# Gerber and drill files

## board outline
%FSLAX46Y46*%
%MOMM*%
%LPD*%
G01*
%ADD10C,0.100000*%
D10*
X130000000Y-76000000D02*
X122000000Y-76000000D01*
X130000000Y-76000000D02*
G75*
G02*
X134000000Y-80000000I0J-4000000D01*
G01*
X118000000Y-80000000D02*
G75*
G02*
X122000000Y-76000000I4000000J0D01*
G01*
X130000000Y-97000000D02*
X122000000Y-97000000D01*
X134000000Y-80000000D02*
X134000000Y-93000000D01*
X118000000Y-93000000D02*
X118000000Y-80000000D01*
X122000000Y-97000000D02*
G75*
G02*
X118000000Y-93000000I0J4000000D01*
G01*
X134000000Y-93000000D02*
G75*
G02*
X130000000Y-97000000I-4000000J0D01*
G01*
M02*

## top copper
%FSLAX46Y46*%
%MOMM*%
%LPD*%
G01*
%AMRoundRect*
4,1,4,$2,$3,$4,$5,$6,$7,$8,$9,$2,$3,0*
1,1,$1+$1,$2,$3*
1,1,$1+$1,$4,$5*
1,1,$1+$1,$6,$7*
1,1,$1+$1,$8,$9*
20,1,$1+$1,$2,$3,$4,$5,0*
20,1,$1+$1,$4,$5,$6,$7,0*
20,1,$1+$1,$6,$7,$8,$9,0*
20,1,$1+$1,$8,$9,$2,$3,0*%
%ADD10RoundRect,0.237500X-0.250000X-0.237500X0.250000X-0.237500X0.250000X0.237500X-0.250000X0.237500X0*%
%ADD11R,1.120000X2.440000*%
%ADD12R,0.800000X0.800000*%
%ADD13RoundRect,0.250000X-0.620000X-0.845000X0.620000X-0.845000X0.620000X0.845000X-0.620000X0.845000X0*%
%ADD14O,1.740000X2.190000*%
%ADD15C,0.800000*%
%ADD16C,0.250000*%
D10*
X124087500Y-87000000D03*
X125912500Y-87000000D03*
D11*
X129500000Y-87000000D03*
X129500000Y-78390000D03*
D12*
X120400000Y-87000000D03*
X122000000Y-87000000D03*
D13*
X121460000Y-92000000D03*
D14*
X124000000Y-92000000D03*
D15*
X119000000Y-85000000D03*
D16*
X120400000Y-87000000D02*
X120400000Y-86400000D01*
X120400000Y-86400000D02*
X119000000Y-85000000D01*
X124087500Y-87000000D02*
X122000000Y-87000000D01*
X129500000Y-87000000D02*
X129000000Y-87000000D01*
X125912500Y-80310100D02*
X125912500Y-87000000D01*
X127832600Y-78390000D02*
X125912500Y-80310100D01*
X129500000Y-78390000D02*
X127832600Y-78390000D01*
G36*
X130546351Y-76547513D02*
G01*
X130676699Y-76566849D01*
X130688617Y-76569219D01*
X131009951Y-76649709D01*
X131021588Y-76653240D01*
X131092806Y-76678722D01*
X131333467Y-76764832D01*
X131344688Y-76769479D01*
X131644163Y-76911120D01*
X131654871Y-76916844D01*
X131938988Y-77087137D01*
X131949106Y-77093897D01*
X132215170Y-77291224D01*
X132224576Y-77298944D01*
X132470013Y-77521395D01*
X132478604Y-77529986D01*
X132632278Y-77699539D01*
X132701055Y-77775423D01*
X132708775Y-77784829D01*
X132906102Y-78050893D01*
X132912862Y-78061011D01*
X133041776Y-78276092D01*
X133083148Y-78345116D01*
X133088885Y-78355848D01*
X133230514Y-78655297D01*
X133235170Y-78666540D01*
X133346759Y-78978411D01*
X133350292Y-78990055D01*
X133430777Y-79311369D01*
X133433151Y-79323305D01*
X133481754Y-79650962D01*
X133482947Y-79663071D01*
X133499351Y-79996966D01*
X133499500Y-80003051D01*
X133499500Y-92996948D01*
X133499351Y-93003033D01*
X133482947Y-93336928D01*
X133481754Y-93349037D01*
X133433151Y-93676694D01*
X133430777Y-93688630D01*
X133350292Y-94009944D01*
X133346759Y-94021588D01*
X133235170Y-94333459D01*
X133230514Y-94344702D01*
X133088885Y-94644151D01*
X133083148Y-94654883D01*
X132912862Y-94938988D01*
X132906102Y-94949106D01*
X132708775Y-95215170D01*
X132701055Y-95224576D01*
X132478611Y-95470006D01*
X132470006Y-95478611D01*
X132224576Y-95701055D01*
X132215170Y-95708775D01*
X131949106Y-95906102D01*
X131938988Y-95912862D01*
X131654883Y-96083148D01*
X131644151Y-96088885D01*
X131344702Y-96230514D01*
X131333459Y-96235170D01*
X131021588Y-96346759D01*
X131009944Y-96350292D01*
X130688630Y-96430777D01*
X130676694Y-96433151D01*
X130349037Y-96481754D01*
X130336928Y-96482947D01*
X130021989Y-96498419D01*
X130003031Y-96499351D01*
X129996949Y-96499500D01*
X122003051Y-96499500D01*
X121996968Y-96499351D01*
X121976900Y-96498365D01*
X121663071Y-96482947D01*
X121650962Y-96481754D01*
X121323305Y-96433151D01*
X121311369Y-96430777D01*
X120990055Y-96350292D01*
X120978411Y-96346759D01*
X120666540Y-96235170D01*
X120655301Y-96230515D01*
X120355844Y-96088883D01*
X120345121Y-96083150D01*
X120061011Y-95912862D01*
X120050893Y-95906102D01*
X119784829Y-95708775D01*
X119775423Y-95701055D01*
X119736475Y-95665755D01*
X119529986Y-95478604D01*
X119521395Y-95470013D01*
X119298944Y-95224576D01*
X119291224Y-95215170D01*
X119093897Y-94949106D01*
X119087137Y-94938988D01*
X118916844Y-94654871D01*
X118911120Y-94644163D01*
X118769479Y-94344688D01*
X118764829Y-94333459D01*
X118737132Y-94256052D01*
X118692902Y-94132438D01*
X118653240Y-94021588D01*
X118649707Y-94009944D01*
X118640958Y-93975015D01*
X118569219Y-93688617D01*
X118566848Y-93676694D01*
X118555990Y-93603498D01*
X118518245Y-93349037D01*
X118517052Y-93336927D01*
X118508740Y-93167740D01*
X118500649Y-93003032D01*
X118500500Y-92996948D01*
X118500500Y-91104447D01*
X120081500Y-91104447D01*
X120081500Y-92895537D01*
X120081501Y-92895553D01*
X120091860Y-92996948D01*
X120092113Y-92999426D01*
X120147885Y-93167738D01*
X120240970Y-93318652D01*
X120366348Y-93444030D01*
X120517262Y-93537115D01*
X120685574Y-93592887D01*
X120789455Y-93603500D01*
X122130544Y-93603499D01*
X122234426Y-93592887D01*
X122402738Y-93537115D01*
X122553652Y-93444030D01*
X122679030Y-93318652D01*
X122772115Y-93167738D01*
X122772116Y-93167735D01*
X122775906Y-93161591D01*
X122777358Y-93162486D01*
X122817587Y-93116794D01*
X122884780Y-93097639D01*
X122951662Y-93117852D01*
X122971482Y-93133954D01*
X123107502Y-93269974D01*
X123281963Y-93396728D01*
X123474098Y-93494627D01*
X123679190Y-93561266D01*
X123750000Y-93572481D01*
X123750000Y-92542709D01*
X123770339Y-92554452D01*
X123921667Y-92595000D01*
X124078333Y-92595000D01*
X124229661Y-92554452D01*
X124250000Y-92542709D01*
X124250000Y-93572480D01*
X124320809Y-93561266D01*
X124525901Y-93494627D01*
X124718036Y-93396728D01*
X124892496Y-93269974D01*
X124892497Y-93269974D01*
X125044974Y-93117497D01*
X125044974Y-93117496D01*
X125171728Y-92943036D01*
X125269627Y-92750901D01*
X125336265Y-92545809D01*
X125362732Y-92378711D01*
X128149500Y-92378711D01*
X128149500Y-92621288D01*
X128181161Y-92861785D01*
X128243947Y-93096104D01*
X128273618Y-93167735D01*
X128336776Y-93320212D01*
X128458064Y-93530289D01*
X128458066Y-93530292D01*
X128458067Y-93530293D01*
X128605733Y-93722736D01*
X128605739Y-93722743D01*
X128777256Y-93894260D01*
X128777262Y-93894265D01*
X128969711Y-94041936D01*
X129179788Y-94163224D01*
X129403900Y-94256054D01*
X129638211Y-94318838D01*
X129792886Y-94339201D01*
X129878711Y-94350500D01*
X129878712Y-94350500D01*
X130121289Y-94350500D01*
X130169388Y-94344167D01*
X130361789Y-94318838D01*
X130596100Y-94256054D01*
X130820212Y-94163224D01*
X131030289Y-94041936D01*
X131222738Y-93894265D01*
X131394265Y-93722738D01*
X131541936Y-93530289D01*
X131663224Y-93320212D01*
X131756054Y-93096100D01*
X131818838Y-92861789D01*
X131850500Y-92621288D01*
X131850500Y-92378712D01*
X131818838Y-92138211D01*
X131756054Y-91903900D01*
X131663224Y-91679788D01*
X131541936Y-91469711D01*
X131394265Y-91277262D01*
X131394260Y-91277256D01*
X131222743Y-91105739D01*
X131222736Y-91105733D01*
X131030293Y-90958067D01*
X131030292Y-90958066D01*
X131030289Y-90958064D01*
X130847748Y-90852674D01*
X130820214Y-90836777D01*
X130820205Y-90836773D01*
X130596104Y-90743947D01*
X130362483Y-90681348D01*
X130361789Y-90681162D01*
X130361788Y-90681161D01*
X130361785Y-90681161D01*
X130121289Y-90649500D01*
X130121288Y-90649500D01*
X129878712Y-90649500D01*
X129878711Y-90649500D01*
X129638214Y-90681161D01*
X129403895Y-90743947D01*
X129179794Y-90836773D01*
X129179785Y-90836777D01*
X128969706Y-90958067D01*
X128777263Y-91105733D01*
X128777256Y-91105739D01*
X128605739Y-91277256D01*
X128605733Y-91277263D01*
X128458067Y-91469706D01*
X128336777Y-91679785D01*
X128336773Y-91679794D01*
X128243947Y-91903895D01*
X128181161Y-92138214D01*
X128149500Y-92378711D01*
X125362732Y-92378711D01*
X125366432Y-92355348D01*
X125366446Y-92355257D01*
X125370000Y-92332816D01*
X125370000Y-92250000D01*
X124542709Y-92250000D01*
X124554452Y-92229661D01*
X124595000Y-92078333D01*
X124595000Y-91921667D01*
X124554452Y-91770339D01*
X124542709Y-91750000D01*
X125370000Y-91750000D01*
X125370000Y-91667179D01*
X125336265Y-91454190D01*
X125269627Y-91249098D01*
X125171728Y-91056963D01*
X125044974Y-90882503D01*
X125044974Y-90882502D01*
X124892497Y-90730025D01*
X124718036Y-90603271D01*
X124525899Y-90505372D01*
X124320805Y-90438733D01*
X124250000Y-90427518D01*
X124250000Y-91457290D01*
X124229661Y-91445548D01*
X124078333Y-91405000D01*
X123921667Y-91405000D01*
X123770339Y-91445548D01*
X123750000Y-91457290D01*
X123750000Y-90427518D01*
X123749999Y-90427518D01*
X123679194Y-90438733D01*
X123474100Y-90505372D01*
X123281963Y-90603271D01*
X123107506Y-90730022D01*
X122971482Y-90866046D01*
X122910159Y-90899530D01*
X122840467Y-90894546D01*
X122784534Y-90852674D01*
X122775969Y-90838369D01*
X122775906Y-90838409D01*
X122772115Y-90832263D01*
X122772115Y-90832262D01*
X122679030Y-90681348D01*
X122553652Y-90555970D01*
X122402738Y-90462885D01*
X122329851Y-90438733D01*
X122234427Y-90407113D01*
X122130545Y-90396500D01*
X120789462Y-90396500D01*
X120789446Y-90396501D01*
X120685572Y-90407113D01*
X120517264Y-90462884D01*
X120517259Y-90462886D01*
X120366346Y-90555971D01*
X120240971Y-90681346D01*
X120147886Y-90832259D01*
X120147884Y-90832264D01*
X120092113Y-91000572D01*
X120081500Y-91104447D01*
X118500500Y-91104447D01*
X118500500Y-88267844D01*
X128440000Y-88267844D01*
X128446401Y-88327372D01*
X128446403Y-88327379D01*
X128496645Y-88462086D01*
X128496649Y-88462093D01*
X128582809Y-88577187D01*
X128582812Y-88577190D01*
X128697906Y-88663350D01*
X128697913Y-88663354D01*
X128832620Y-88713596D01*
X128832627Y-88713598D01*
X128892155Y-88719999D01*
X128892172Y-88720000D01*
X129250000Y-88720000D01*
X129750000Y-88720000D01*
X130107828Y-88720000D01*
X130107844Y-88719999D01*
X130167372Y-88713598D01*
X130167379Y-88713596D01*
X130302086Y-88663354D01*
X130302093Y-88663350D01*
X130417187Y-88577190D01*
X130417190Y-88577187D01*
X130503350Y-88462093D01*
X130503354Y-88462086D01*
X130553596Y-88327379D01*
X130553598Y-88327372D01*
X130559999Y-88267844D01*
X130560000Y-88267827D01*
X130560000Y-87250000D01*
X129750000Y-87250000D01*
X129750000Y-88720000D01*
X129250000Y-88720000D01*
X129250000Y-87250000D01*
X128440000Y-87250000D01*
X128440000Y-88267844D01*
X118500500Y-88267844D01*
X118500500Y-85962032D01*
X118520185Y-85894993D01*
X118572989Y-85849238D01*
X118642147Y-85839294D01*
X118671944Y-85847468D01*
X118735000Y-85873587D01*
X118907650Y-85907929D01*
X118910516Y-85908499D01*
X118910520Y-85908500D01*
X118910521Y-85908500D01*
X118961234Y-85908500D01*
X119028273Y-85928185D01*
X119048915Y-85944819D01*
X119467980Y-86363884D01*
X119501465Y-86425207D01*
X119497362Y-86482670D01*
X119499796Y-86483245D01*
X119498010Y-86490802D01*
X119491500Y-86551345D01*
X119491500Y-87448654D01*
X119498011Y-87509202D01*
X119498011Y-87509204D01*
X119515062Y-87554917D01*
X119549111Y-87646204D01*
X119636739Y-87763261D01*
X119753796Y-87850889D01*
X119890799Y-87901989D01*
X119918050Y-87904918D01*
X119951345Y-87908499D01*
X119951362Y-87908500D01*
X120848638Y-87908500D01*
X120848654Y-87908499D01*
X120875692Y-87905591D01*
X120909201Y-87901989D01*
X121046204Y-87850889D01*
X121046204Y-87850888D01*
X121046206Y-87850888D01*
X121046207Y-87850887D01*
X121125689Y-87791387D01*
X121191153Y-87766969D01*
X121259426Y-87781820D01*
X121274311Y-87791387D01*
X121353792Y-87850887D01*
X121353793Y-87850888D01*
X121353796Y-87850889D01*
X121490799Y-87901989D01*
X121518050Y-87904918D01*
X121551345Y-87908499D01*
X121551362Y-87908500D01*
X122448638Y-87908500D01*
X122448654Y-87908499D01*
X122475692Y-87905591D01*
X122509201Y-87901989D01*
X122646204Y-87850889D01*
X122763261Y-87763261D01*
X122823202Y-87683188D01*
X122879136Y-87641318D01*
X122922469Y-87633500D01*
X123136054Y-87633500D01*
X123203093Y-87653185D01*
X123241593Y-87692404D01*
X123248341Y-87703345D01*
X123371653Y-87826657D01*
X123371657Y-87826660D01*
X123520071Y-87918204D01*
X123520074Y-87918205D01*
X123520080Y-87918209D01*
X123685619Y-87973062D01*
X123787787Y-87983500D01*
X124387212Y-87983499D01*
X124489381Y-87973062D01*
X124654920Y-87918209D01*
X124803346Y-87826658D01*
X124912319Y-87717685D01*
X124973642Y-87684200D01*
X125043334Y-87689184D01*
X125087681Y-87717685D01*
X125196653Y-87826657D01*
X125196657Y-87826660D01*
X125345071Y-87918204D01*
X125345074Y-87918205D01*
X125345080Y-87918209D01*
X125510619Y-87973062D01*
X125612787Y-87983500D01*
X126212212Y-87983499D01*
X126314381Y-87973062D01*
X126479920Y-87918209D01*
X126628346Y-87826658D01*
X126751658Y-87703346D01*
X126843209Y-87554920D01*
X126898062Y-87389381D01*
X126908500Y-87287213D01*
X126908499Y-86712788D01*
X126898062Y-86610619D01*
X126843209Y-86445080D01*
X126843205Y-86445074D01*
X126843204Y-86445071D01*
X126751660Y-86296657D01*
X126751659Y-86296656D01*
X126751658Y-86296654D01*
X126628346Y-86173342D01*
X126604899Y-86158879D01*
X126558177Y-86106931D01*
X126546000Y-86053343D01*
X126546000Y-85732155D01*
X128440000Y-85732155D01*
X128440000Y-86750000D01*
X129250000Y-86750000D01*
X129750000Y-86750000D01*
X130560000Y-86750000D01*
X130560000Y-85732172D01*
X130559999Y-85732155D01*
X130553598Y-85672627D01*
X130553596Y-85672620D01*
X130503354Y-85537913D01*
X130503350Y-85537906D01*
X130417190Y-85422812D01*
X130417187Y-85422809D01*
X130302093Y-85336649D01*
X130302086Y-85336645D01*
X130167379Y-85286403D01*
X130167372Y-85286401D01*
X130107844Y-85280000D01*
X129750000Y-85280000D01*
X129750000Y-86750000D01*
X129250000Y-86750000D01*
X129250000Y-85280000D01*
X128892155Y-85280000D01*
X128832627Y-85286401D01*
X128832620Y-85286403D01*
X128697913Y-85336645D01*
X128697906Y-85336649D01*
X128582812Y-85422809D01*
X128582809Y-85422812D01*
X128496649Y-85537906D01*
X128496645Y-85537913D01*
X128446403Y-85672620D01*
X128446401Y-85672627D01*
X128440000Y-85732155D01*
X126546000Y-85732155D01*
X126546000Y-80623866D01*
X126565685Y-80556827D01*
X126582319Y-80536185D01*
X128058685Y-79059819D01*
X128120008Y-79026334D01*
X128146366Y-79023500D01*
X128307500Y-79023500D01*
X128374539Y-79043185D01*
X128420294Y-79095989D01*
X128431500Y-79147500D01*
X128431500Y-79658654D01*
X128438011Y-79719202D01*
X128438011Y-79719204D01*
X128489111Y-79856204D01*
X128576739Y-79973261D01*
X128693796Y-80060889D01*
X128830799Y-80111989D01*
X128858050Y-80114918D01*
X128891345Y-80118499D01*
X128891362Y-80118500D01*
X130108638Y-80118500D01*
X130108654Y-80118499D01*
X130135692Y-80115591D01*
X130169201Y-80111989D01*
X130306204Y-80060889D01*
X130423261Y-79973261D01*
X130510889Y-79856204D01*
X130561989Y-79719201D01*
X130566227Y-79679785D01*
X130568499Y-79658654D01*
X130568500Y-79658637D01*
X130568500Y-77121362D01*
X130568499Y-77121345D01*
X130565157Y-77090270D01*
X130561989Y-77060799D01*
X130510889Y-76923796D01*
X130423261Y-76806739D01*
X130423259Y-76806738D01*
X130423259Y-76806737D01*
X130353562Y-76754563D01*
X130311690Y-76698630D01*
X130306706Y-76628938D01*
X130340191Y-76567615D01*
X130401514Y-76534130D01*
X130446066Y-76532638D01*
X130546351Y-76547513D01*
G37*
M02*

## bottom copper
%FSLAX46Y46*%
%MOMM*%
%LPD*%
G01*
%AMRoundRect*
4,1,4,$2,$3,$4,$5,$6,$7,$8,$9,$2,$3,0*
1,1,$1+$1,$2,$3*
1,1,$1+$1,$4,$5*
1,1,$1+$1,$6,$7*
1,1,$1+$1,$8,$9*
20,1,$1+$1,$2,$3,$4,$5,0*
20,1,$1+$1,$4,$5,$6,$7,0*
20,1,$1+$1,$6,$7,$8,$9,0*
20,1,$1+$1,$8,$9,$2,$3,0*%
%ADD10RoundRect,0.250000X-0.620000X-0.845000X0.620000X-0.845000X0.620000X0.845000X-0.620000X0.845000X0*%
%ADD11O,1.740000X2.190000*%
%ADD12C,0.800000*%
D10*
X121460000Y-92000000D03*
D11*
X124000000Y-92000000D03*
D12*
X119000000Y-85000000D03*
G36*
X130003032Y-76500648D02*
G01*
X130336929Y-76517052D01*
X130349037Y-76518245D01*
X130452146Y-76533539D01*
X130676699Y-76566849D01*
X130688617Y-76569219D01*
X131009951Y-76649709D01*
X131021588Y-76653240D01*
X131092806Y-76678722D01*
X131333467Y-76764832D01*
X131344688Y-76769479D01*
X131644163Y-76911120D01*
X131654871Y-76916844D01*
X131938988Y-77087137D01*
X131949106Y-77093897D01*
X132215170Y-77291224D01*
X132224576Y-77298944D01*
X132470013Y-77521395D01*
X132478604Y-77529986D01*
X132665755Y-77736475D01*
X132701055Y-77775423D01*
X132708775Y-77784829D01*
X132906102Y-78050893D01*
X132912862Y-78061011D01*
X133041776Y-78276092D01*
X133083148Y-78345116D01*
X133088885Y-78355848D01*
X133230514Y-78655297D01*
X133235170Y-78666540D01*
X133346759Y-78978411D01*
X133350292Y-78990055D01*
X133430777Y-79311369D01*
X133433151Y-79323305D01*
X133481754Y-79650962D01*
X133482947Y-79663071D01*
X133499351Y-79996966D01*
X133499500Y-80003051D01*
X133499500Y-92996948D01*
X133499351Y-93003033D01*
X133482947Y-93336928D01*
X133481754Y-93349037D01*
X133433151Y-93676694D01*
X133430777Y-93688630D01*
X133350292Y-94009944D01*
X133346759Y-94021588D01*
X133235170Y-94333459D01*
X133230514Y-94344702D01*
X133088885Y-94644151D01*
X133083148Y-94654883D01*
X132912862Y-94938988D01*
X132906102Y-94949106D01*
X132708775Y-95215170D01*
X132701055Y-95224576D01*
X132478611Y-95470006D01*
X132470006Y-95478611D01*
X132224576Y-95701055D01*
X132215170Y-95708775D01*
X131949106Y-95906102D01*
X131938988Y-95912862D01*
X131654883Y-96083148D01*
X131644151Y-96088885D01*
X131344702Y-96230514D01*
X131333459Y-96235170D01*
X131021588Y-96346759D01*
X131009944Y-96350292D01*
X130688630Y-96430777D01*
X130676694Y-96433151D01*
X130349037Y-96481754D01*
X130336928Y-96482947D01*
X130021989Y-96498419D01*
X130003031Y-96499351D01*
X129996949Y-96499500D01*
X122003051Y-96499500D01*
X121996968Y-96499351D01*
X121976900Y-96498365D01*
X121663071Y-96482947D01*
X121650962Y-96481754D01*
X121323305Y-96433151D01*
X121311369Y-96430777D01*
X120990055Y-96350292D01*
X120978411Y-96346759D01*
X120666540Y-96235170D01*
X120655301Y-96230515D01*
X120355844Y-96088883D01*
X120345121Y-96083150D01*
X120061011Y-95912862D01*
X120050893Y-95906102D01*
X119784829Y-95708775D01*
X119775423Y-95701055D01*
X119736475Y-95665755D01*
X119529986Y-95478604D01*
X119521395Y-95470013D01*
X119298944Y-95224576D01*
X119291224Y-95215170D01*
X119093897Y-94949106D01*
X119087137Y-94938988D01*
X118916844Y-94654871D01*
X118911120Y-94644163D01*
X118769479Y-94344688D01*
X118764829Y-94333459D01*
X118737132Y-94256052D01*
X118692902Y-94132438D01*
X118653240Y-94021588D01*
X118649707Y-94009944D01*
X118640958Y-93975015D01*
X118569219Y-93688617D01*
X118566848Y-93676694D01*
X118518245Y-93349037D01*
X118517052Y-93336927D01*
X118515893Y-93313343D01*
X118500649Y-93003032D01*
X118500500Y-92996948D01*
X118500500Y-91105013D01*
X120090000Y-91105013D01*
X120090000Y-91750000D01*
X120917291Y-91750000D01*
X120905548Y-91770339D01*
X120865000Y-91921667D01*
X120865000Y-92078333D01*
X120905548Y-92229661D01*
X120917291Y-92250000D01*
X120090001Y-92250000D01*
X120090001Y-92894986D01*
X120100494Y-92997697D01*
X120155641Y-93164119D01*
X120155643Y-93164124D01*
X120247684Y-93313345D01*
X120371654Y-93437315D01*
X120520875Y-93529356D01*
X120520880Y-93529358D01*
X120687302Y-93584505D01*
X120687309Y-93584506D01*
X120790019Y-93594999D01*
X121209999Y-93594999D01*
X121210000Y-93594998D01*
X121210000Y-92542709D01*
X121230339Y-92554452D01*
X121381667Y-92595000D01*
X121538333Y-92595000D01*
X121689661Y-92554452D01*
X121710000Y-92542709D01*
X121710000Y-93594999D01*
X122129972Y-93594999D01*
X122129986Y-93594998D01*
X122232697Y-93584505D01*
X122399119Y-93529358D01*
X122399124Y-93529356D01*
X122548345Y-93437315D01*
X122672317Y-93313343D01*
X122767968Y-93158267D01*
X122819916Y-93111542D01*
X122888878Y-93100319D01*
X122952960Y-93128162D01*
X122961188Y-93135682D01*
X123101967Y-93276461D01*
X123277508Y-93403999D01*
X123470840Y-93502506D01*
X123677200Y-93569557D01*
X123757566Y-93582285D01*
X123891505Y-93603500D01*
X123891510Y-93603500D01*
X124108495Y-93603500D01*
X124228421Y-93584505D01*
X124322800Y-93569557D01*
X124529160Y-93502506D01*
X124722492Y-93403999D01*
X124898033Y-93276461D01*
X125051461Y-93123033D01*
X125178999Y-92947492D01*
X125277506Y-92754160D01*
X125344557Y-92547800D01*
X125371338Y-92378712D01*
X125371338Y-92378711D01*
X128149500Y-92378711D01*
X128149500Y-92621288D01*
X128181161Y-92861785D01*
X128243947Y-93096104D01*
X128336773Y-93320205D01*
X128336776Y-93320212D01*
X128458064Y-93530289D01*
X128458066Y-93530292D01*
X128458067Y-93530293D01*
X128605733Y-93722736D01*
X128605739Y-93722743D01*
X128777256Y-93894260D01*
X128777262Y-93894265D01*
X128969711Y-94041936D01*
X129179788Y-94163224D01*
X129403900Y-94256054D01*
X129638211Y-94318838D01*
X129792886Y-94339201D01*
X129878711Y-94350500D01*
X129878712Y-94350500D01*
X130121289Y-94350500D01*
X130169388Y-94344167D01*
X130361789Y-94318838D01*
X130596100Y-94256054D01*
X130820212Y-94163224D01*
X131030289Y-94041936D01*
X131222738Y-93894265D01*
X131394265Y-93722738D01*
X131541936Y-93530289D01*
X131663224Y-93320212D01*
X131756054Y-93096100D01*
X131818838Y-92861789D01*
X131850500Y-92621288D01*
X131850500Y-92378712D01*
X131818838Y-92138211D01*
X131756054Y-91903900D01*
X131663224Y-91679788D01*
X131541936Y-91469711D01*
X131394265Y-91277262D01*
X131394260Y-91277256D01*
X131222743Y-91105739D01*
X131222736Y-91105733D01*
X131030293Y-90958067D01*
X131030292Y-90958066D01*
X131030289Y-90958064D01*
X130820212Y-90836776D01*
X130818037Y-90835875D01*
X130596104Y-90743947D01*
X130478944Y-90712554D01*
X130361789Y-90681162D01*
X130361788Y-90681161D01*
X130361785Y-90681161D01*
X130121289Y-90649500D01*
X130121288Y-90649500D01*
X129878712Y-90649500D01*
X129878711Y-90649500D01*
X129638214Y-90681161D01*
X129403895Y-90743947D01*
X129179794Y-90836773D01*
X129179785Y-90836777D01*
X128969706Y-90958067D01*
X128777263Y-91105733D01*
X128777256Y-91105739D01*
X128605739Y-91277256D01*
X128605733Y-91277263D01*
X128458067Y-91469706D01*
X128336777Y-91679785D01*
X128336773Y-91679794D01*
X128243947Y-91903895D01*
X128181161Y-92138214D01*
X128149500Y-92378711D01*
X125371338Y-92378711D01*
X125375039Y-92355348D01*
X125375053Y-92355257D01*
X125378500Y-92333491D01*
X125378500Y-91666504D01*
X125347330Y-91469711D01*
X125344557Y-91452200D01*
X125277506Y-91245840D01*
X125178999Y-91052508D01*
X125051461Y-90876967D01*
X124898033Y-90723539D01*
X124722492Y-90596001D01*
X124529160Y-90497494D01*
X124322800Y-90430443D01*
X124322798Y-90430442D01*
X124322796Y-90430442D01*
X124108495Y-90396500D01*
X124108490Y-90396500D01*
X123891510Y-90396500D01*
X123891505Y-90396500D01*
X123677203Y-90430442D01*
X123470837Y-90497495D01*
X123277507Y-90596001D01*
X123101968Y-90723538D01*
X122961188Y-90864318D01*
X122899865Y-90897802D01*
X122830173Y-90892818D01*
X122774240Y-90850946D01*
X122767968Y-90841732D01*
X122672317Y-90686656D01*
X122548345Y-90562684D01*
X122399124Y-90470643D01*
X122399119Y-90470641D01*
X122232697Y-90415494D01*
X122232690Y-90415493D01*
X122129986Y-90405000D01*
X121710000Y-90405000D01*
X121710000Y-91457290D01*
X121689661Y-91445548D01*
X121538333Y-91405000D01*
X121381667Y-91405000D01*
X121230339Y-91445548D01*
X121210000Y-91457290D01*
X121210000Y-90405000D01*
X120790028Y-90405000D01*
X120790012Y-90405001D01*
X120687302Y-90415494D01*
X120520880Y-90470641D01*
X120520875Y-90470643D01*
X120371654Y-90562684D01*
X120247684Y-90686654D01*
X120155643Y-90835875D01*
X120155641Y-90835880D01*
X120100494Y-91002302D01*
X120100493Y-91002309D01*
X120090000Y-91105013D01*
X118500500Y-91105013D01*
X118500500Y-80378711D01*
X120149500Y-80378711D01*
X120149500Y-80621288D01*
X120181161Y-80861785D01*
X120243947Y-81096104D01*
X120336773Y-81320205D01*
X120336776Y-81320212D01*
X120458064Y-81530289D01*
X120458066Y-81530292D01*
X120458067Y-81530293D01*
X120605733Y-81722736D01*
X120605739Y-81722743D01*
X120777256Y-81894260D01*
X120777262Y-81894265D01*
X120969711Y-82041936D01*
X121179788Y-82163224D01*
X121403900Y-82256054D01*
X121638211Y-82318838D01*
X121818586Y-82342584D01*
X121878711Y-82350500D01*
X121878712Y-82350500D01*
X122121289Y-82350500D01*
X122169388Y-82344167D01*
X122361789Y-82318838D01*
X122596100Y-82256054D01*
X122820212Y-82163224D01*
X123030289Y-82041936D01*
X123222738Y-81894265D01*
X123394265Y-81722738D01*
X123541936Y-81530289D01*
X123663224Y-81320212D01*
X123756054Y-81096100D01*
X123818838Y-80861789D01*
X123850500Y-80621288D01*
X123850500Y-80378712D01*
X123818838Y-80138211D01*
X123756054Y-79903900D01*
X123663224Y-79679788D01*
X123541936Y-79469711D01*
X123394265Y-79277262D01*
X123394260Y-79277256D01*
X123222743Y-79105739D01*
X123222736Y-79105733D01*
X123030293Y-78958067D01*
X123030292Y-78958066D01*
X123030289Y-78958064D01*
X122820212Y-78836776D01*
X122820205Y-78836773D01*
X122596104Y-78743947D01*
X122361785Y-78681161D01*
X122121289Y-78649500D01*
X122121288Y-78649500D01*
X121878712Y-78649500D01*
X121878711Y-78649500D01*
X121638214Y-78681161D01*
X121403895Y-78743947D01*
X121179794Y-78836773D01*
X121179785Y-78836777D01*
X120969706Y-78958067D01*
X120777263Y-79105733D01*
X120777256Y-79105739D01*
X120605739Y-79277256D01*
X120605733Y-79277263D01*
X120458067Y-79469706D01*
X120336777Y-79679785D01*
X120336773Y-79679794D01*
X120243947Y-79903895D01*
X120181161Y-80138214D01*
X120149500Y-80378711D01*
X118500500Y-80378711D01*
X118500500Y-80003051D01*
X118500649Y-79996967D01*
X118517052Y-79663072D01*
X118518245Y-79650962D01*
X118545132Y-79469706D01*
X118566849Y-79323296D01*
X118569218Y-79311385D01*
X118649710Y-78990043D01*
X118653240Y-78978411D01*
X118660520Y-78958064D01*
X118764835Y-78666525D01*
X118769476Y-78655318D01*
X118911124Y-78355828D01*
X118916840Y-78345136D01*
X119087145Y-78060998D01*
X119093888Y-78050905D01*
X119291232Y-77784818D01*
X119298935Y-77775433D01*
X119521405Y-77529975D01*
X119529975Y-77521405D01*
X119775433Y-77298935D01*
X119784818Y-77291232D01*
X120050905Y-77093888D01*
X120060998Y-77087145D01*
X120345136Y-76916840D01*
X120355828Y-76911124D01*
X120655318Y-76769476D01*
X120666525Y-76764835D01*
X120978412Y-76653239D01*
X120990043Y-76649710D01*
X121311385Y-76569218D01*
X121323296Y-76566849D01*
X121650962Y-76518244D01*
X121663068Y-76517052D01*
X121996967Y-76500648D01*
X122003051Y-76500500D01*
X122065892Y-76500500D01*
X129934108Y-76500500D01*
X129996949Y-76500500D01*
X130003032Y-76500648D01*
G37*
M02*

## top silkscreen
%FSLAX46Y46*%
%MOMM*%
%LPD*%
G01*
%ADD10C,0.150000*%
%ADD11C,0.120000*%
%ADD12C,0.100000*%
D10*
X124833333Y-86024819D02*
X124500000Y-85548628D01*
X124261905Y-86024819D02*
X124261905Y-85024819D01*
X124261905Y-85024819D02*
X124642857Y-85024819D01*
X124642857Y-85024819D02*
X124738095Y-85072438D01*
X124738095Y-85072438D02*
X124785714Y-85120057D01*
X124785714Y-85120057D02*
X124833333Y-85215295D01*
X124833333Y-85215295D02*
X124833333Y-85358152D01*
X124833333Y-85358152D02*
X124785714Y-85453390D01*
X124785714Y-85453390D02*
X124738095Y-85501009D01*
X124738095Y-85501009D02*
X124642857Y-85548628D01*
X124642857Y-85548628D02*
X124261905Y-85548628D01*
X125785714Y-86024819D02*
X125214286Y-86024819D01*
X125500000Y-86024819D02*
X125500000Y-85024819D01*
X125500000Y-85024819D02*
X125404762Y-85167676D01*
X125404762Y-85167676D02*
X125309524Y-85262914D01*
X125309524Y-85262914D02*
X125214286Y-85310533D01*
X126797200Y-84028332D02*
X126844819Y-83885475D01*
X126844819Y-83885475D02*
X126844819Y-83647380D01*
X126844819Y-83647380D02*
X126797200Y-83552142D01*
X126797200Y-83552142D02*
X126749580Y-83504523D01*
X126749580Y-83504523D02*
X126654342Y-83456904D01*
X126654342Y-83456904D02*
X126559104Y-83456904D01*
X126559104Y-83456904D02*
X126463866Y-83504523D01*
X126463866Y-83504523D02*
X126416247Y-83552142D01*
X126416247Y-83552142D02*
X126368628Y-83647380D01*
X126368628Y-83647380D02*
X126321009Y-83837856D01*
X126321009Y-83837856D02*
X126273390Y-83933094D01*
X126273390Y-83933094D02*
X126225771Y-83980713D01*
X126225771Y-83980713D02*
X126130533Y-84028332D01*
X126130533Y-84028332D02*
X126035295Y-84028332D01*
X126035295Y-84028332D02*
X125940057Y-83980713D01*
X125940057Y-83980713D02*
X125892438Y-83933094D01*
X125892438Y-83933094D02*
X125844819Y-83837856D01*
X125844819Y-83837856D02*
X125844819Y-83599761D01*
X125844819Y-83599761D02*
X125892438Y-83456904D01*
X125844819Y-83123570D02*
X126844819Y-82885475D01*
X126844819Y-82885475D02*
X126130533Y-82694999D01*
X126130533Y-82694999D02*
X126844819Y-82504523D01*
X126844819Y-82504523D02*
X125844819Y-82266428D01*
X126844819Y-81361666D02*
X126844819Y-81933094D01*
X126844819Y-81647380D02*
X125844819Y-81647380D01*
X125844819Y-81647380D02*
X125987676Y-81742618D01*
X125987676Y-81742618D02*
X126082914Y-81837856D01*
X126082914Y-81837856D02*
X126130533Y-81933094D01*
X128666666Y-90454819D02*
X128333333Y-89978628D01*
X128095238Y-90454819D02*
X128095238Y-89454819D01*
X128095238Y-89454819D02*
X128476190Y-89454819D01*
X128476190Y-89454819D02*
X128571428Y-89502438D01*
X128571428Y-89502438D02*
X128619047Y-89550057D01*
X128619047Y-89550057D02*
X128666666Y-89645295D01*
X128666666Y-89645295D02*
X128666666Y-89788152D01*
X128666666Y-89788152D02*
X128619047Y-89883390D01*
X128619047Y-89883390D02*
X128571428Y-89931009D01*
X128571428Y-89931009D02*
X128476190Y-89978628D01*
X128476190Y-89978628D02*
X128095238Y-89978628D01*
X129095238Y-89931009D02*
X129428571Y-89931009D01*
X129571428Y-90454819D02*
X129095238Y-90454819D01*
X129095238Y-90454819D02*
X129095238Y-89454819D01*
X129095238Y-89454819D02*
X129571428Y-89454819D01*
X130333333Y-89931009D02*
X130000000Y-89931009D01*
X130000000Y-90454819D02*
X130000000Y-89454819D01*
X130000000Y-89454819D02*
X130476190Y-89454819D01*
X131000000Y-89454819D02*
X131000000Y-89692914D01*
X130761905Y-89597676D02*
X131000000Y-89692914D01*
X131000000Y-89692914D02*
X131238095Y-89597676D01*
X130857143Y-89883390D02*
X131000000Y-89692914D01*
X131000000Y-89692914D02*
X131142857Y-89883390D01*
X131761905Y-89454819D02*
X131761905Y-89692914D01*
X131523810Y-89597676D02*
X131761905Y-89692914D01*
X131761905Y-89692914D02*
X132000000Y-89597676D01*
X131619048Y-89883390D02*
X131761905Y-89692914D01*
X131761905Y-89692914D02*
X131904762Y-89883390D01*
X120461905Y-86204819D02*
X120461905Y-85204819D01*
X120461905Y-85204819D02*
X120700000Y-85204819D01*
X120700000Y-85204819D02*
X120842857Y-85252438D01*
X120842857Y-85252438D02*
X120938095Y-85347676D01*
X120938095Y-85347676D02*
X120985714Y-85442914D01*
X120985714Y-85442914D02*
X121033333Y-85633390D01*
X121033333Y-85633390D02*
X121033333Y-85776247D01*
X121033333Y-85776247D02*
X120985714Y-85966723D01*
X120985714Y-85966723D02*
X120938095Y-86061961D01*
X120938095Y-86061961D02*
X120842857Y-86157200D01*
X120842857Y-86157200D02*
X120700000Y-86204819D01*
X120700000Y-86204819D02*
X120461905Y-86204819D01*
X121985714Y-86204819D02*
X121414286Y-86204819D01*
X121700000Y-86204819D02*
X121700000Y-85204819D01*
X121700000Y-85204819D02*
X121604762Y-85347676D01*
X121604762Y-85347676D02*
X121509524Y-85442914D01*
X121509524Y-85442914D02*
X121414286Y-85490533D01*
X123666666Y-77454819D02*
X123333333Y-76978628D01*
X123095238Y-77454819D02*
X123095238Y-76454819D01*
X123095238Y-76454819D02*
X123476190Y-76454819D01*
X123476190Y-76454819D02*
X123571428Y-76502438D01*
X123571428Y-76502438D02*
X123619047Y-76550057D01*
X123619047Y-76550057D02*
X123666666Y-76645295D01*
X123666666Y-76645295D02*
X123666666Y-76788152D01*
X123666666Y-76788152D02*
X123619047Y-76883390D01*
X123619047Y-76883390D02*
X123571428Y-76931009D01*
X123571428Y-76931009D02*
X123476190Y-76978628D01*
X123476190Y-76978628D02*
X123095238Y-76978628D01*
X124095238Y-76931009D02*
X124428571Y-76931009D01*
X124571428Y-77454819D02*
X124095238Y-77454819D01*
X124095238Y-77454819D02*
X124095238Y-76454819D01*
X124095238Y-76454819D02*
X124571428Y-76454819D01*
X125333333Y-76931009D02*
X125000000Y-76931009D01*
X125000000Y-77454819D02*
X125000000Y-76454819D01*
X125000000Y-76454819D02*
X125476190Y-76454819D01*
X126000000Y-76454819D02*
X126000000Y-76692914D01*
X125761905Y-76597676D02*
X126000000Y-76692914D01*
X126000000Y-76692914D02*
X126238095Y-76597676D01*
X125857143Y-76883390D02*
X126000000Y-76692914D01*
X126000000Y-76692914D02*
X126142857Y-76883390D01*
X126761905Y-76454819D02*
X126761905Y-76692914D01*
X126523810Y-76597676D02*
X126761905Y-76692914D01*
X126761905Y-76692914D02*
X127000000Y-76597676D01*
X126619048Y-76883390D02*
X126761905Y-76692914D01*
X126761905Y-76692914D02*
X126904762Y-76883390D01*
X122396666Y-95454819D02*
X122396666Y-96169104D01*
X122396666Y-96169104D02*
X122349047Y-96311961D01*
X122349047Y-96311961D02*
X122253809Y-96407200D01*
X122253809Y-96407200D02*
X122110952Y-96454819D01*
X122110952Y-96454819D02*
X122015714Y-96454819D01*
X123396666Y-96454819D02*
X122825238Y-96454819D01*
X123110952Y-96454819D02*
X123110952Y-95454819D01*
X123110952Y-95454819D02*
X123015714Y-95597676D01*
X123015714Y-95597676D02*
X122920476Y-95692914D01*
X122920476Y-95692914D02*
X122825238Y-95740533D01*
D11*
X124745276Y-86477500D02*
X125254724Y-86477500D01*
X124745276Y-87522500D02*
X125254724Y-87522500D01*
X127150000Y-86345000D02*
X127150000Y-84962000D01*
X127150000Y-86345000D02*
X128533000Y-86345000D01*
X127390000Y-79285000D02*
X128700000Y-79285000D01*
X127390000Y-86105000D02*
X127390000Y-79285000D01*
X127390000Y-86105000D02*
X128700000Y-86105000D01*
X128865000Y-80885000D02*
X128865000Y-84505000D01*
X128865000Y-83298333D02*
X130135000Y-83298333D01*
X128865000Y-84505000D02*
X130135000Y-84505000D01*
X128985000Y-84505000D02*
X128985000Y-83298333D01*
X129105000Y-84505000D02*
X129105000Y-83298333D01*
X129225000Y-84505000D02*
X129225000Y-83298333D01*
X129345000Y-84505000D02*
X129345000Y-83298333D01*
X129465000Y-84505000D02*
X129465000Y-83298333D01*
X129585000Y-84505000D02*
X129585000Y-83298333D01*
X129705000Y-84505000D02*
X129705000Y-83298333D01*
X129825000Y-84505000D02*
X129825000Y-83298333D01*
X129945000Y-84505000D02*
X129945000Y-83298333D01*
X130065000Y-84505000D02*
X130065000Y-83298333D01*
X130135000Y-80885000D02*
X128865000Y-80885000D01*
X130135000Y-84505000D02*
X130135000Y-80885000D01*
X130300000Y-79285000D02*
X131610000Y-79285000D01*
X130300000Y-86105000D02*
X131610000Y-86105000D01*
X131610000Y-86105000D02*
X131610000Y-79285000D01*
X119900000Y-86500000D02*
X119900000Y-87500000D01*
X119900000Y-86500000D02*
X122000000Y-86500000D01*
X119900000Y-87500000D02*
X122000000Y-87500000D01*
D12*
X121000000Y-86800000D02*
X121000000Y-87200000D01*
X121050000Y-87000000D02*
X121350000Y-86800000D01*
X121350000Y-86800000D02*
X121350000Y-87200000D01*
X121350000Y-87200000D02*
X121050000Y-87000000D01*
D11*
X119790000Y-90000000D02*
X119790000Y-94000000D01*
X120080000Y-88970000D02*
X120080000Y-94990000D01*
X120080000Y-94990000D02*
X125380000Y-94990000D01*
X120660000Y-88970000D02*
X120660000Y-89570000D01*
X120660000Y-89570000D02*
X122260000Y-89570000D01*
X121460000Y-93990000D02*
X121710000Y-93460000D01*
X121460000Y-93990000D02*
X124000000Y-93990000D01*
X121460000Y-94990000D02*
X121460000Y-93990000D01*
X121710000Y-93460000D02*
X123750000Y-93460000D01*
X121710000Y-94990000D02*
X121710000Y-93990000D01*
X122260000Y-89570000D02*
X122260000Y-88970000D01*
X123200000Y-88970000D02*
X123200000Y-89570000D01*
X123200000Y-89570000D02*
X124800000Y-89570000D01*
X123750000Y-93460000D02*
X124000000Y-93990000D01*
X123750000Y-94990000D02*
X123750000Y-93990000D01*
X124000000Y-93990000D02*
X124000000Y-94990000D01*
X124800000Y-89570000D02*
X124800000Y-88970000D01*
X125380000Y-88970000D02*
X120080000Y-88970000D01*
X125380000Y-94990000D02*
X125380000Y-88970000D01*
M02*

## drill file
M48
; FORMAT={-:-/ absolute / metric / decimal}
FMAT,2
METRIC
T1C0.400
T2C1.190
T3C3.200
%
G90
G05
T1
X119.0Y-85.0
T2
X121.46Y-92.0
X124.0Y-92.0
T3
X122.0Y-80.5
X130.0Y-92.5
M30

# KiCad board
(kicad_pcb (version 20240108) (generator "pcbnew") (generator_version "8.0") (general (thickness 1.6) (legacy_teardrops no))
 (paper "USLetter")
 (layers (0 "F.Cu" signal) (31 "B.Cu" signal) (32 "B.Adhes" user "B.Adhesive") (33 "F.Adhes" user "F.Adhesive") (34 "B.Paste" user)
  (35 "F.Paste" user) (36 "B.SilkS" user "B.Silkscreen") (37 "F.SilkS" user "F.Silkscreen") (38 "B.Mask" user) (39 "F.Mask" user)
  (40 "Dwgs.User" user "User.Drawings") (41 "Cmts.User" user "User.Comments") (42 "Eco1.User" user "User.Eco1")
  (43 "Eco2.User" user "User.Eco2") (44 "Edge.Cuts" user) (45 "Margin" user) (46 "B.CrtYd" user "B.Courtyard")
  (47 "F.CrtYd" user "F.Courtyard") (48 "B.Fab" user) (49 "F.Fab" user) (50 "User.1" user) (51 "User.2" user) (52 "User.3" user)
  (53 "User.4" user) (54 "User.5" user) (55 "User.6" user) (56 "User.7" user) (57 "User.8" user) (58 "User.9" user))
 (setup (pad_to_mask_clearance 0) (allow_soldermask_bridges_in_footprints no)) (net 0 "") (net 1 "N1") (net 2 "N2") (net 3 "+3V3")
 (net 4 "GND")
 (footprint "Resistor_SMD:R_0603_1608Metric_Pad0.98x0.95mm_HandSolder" (layer "F.Cu") (at 125 87)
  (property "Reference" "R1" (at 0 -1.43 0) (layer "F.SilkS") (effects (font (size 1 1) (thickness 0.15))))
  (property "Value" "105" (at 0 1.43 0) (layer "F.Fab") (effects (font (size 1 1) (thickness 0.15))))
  (fp_line (start -0.254724 -0.5225) (end 0.254724 -0.5225) (stroke (width 0.12) (type solid)) (layer "F.SilkS"))
  (fp_line (start -0.254724 0.5225) (end 0.254724 0.5225) (stroke (width 0.12) (type solid)) (layer "F.SilkS"))
  (pad "1" smd roundrect (at -0.9125 0) (size 0.975 0.95) (layers "F.Cu" "F.Paste" "F.Mask") (roundrect_rratio 0.25) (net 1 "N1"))
  (pad "2" smd roundrect (at 0.9125 0) (size 0.975 0.95) (layers "F.Cu" "F.Paste" "F.Mask") (roundrect_rratio 0.25) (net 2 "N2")))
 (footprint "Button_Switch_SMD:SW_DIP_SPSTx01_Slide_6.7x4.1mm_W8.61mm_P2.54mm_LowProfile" (layer "F.Cu") (at 129.5 82.695 90)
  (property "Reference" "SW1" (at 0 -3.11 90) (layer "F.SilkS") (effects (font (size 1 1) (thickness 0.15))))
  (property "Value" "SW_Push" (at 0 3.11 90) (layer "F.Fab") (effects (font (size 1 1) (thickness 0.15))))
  (fp_line (start -3.65 -2.35) (end -2.267 -2.35) (stroke (width 0.12) (type solid)) (layer "F.SilkS"))
  (fp_line (start -3.65 -2.35) (end -3.65 -0.967) (stroke (width 0.12) (type solid)) (layer "F.SilkS"))
  (fp_line (start 3.41 -2.11) (end 3.41 -0.8) (stroke (width 0.12) (type solid)) (layer "F.SilkS"))
  (fp_line (start -3.41 -2.11) (end 3.41 -2.11) (stroke (width 0.12) (type solid)) (layer "F.SilkS"))
  (fp_line (start -3.41 -2.11) (end -3.41 -0.8) (stroke (width 0.12) (type solid)) (layer "F.SilkS"))
  (fp_line (start 1.81 -0.635) (end -1.81 -0.635) (stroke (width 0.12) (type solid)) (layer "F.SilkS"))
  (fp_line (start -0.603333 -0.635) (end -0.603333 0.635) (stroke (width 0.12) (type solid)) (layer "F.SilkS"))
  (fp_line (start -1.81 -0.635) (end -1.81 0.635) (stroke (width 0.12) (type solid)) (layer "F.SilkS"))
  (fp_line (start -1.81 -0.515) (end -0.603333 -0.515) (stroke (width 0.12) (type solid)) (layer "F.SilkS"))
  (fp_line (start -1.81 -0.395) (end -0.603333 -0.395) (stroke (width 0.12) (type solid)) (layer "F.SilkS"))
  (fp_line (start -1.81 -0.275) (end -0.603333 -0.275) (stroke (width 0.12) (type solid)) (layer "F.SilkS"))
  (fp_line (start -1.81 -0.155) (end -0.603333 -0.155) (stroke (width 0.12) (type solid)) (layer "F.SilkS"))
  (fp_line (start -1.81 -0.035) (end -0.603333 -0.035) (stroke (width 0.12) (type solid)) (layer "F.SilkS"))
  (fp_line (start -1.81 0.085) (end -0.603333 0.085) (stroke (width 0.12) (type solid)) (layer "F.SilkS"))
  (fp_line (start -1.81 0.205) (end -0.603333 0.205) (stroke (width 0.12) (type solid)) (layer "F.SilkS"))
  (fp_line (start -1.81 0.325) (end -0.603333 0.325) (stroke (width 0.12) (type solid)) (layer "F.SilkS"))
  (fp_line (start -1.81 0.445) (end -0.603333 0.445) (stroke (width 0.12) (type solid)) (layer "F.SilkS"))
  (fp_line (start -1.81 0.565) (end -0.603333 0.565) (stroke (width 0.12) (type solid)) (layer "F.SilkS"))
  (fp_line (start 1.81 0.635) (end 1.81 -0.635) (stroke (width 0.12) (type solid)) (layer "F.SilkS"))
  (fp_line (start -1.81 0.635) (end 1.81 0.635) (stroke (width 0.12) (type solid)) (layer "F.SilkS"))
  (fp_line (start 3.41 0.8) (end 3.41 2.11) (stroke (width 0.12) (type solid)) (layer "F.SilkS"))
  (fp_line (start -3.41 0.8) (end -3.41 2.11) (stroke (width 0.12) (type solid)) (layer "F.SilkS"))
  (fp_line (start -3.41 2.11) (end 3.41 2.11) (stroke (width 0.12) (type solid)) (layer "F.SilkS"))
  (pad "1" smd rect (at -4.305 0 90) (size 2.44 1.12) (layers "F.Cu" "F.Paste" "F.Mask") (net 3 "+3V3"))
  (pad "2" smd rect (at 4.305 0 90) (size 2.44 1.12) (layers "F.Cu" "F.Paste" "F.Mask") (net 2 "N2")))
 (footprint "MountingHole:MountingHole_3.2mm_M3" (layer "F.Cu") (at 130 92.5)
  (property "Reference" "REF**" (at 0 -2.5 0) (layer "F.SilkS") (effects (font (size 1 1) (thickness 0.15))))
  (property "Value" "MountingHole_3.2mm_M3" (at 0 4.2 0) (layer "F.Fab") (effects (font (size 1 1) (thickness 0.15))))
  (pad "" np_thru_hole circle (at 0 0) (size 3.2 3.2) (drill 3.2) (layers "*.Cu" "*.Mask")))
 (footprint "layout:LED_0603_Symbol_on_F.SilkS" (layer "F.Cu") (at 121.2 87)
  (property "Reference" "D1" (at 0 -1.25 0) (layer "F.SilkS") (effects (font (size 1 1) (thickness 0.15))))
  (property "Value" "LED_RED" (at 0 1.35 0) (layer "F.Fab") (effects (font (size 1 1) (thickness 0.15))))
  (fp_line (start -1.3 -0.5) (end -1.3 0.5) (stroke (width 0.12) (type solid)) (layer "F.SilkS"))
  (fp_line (start -1.3 -0.5) (end 0.8 -0.5) (stroke (width 0.12) (type solid)) (layer "F.SilkS"))
  (fp_line (start -1.3 0.5) (end 0.8 0.5) (stroke (width 0.12) (type solid)) (layer "F.SilkS"))
  (fp_line (start -0.2 -0.2) (end -0.2 0.2) (stroke (width 0.1) (type solid)) (layer "F.SilkS"))
  (fp_line (start -0.15 0) (end 0.15 -0.2) (stroke (width 0.1) (type solid)) (layer "F.SilkS"))
  (fp_line (start 0.15 -0.2) (end 0.15 0.2) (stroke (width 0.1) (type solid)) (layer "F.SilkS"))
  (fp_line (start 0.15 0.2) (end -0.15 0) (stroke (width 0.1) (type solid)) (layer "F.SilkS"))
  (pad "1" smd rect (at -0.8 0 180) (size 0.8 0.8) (layers "F.Cu" "F.Paste" "F.Mask") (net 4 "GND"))
  (pad "2" smd rect (at 0.8 0 180) (size 0.8 0.8) (layers "F.Cu" "F.Paste" "F.Mask") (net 1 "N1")))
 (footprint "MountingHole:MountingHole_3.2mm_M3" (layer "F.Cu") (at 122 80.5)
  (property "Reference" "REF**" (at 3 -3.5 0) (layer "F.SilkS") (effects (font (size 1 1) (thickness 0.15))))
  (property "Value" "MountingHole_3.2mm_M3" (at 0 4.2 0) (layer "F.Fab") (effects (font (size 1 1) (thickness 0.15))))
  (pad "" np_thru_hole circle (at 0 0) (size 3.2 3.2) (drill 3.2) (layers "*.Cu" "*.Mask")))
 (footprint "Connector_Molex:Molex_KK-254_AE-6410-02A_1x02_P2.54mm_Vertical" (layer "F.Cu") (at 121.46 92)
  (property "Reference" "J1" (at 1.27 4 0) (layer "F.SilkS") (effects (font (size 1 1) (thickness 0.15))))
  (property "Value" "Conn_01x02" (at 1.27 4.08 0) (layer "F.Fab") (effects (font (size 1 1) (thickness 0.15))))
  (fp_line (start -1.67 -2) (end -1.67 2) (stroke (width 0.12) (type solid)) (layer "F.SilkS"))
  (fp_line (start -1.38 -3.03) (end -1.38 2.99) (stroke (width 0.12) (type solid)) (layer "F.SilkS"))
  (fp_line (start -1.38 2.99) (end 3.92 2.99) (stroke (width 0.12) (type solid)) (layer "F.SilkS"))
  (fp_line (start -0.8 -3.03) (end -0.8 -2.43) (stroke (width 0.12) (type solid)) (layer "F.SilkS"))
  (fp_line (start -0.8 -2.43) (end 0.8 -2.43) (stroke (width 0.12) (type solid)) (layer "F.SilkS"))
  (fp_line (start 0 1.99) (end 0.25 1.46) (stroke (width 0.12) (type solid)) (layer "F.SilkS"))
  (fp_line (start 0 1.99) (end 2.54 1.99) (stroke (width 0.12) (type solid)) (layer "F.SilkS"))
  (fp_line (start 0 2.99) (end 0 1.99) (stroke (width 0.12) (type solid)) (layer "F.SilkS"))
  (fp_line (start 0.25 1.46) (end 2.29 1.46) (stroke (width 0.12) (type solid)) (layer "F.SilkS"))
  (fp_line (start 0.25 2.99) (end 0.25 1.99) (stroke (width 0.12) (type solid)) (layer "F.SilkS"))
  (fp_line (start 0.8 -2.43) (end 0.8 -3.03) (stroke (width 0.12) (type solid)) (layer "F.SilkS"))
  (fp_line (start 1.74 -3.03) (end 1.74 -2.43) (stroke (width 0.12) (type solid)) (layer "F.SilkS"))
  (fp_line (start 1.74 -2.43) (end 3.34 -2.43) (stroke (width 0.12) (type solid)) (layer "F.SilkS"))
  (fp_line (start 2.29 1.46) (end 2.54 1.99) (stroke (width 0.12) (type solid)) (layer "F.SilkS"))
  (fp_line (start 2.29 2.99) (end 2.29 1.99) (stroke (width 0.12) (type solid)) (layer "F.SilkS"))
  (fp_line (start 2.54 1.99) (end 2.54 2.99) (stroke (width 0.12) (type solid)) (layer "F.SilkS"))
  (fp_line (start 3.34 -2.43) (end 3.34 -3.03) (stroke (width 0.12) (type solid)) (layer "F.SilkS"))
  (fp_line (start 3.92 -3.03) (end -1.38 -3.03) (stroke (width 0.12) (type solid)) (layer "F.SilkS"))
  (fp_line (start 3.92 2.99) (end 3.92 -3.03) (stroke (width 0.12) (type solid)) (layer "F.SilkS"))
  (pad "1" thru_hole roundrect (at 0 0) (size 1.74 2.19) (drill 1.19) (layers "*.Cu" "*.Mask") (remove_unused_layers no)
   (roundrect_rratio 0.143678) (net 4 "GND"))
  (pad "2" thru_hole oval (at 2.54 0) (size 1.74 2.19) (drill 1.19) (layers "*.Cu" "*.Mask") (remove_unused_layers no) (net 3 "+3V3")))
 (gr_line (start 130 76) (end 122 76) (stroke (width 0.1) (type default)) (layer "Edge.Cuts"))
 (gr_arc (start 130 76) (mid 132.828427 77.171573) (end 134 80) (stroke (width 0.1) (type default)) (layer "Edge.Cuts"))
 (gr_arc (start 118 80) (mid 119.171573 77.171573) (end 122 76) (stroke (width 0.1) (type default)) (layer "Edge.Cuts"))
 (gr_line (start 130 97) (end 122 97) (stroke (width 0.1) (type default)) (layer "Edge.Cuts"))
 (gr_line (start 134 80) (end 134 93) (stroke (width 0.1) (type default)) (layer "Edge.Cuts"))
 (gr_line (start 118 93) (end 118 80) (stroke (width 0.1) (type default)) (layer "Edge.Cuts"))
 (gr_arc (start 122 97) (mid 119.171573 95.828427) (end 118 93) (stroke (width 0.1) (type default)) (layer "Edge.Cuts"))
 (gr_arc (start 134 93) (mid 132.828427 95.828427) (end 130 97) (stroke (width 0.1) (type default)) (layer "Edge.Cuts"))
 (segment (start 120.4 87) (end 120.4 86.4) (width 0.25) (layer "F.Cu") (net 4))
 (segment (start 120.4 86.4) (end 119 85) (width 0.25) (layer "F.Cu") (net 4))
 (via (at 119 85) (size 0.8) (drill 0.4) (layers "F.Cu" "B.Cu") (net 4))
 (segment (start 124.0875 87) (end 122 87) (width 0.25) (layer "F.Cu") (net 1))
 (segment (start 129.5 87) (end 129 87) (width 0.25) (layer "F.Cu") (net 3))
 (segment (start 125.9125 80.3101) (end 125.9125 87) (width 0.25) (layer "F.Cu") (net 2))
 (segment (start 127.8326 78.39) (end 125.9125 80.3101) (width 0.25) (layer "F.Cu") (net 2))
 (segment (start 129.5 78.39) (end 127.8326 78.39) (width 0.25) (layer "F.Cu") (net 2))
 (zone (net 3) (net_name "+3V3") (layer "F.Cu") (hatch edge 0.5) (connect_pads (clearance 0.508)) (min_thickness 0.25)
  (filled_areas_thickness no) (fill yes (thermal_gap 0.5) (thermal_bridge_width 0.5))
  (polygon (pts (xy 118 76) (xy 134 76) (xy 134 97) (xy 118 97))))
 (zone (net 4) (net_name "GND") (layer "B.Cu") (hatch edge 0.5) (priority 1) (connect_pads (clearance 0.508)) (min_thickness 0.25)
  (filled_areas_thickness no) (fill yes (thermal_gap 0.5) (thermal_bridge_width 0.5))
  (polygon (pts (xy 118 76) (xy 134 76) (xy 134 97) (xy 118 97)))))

